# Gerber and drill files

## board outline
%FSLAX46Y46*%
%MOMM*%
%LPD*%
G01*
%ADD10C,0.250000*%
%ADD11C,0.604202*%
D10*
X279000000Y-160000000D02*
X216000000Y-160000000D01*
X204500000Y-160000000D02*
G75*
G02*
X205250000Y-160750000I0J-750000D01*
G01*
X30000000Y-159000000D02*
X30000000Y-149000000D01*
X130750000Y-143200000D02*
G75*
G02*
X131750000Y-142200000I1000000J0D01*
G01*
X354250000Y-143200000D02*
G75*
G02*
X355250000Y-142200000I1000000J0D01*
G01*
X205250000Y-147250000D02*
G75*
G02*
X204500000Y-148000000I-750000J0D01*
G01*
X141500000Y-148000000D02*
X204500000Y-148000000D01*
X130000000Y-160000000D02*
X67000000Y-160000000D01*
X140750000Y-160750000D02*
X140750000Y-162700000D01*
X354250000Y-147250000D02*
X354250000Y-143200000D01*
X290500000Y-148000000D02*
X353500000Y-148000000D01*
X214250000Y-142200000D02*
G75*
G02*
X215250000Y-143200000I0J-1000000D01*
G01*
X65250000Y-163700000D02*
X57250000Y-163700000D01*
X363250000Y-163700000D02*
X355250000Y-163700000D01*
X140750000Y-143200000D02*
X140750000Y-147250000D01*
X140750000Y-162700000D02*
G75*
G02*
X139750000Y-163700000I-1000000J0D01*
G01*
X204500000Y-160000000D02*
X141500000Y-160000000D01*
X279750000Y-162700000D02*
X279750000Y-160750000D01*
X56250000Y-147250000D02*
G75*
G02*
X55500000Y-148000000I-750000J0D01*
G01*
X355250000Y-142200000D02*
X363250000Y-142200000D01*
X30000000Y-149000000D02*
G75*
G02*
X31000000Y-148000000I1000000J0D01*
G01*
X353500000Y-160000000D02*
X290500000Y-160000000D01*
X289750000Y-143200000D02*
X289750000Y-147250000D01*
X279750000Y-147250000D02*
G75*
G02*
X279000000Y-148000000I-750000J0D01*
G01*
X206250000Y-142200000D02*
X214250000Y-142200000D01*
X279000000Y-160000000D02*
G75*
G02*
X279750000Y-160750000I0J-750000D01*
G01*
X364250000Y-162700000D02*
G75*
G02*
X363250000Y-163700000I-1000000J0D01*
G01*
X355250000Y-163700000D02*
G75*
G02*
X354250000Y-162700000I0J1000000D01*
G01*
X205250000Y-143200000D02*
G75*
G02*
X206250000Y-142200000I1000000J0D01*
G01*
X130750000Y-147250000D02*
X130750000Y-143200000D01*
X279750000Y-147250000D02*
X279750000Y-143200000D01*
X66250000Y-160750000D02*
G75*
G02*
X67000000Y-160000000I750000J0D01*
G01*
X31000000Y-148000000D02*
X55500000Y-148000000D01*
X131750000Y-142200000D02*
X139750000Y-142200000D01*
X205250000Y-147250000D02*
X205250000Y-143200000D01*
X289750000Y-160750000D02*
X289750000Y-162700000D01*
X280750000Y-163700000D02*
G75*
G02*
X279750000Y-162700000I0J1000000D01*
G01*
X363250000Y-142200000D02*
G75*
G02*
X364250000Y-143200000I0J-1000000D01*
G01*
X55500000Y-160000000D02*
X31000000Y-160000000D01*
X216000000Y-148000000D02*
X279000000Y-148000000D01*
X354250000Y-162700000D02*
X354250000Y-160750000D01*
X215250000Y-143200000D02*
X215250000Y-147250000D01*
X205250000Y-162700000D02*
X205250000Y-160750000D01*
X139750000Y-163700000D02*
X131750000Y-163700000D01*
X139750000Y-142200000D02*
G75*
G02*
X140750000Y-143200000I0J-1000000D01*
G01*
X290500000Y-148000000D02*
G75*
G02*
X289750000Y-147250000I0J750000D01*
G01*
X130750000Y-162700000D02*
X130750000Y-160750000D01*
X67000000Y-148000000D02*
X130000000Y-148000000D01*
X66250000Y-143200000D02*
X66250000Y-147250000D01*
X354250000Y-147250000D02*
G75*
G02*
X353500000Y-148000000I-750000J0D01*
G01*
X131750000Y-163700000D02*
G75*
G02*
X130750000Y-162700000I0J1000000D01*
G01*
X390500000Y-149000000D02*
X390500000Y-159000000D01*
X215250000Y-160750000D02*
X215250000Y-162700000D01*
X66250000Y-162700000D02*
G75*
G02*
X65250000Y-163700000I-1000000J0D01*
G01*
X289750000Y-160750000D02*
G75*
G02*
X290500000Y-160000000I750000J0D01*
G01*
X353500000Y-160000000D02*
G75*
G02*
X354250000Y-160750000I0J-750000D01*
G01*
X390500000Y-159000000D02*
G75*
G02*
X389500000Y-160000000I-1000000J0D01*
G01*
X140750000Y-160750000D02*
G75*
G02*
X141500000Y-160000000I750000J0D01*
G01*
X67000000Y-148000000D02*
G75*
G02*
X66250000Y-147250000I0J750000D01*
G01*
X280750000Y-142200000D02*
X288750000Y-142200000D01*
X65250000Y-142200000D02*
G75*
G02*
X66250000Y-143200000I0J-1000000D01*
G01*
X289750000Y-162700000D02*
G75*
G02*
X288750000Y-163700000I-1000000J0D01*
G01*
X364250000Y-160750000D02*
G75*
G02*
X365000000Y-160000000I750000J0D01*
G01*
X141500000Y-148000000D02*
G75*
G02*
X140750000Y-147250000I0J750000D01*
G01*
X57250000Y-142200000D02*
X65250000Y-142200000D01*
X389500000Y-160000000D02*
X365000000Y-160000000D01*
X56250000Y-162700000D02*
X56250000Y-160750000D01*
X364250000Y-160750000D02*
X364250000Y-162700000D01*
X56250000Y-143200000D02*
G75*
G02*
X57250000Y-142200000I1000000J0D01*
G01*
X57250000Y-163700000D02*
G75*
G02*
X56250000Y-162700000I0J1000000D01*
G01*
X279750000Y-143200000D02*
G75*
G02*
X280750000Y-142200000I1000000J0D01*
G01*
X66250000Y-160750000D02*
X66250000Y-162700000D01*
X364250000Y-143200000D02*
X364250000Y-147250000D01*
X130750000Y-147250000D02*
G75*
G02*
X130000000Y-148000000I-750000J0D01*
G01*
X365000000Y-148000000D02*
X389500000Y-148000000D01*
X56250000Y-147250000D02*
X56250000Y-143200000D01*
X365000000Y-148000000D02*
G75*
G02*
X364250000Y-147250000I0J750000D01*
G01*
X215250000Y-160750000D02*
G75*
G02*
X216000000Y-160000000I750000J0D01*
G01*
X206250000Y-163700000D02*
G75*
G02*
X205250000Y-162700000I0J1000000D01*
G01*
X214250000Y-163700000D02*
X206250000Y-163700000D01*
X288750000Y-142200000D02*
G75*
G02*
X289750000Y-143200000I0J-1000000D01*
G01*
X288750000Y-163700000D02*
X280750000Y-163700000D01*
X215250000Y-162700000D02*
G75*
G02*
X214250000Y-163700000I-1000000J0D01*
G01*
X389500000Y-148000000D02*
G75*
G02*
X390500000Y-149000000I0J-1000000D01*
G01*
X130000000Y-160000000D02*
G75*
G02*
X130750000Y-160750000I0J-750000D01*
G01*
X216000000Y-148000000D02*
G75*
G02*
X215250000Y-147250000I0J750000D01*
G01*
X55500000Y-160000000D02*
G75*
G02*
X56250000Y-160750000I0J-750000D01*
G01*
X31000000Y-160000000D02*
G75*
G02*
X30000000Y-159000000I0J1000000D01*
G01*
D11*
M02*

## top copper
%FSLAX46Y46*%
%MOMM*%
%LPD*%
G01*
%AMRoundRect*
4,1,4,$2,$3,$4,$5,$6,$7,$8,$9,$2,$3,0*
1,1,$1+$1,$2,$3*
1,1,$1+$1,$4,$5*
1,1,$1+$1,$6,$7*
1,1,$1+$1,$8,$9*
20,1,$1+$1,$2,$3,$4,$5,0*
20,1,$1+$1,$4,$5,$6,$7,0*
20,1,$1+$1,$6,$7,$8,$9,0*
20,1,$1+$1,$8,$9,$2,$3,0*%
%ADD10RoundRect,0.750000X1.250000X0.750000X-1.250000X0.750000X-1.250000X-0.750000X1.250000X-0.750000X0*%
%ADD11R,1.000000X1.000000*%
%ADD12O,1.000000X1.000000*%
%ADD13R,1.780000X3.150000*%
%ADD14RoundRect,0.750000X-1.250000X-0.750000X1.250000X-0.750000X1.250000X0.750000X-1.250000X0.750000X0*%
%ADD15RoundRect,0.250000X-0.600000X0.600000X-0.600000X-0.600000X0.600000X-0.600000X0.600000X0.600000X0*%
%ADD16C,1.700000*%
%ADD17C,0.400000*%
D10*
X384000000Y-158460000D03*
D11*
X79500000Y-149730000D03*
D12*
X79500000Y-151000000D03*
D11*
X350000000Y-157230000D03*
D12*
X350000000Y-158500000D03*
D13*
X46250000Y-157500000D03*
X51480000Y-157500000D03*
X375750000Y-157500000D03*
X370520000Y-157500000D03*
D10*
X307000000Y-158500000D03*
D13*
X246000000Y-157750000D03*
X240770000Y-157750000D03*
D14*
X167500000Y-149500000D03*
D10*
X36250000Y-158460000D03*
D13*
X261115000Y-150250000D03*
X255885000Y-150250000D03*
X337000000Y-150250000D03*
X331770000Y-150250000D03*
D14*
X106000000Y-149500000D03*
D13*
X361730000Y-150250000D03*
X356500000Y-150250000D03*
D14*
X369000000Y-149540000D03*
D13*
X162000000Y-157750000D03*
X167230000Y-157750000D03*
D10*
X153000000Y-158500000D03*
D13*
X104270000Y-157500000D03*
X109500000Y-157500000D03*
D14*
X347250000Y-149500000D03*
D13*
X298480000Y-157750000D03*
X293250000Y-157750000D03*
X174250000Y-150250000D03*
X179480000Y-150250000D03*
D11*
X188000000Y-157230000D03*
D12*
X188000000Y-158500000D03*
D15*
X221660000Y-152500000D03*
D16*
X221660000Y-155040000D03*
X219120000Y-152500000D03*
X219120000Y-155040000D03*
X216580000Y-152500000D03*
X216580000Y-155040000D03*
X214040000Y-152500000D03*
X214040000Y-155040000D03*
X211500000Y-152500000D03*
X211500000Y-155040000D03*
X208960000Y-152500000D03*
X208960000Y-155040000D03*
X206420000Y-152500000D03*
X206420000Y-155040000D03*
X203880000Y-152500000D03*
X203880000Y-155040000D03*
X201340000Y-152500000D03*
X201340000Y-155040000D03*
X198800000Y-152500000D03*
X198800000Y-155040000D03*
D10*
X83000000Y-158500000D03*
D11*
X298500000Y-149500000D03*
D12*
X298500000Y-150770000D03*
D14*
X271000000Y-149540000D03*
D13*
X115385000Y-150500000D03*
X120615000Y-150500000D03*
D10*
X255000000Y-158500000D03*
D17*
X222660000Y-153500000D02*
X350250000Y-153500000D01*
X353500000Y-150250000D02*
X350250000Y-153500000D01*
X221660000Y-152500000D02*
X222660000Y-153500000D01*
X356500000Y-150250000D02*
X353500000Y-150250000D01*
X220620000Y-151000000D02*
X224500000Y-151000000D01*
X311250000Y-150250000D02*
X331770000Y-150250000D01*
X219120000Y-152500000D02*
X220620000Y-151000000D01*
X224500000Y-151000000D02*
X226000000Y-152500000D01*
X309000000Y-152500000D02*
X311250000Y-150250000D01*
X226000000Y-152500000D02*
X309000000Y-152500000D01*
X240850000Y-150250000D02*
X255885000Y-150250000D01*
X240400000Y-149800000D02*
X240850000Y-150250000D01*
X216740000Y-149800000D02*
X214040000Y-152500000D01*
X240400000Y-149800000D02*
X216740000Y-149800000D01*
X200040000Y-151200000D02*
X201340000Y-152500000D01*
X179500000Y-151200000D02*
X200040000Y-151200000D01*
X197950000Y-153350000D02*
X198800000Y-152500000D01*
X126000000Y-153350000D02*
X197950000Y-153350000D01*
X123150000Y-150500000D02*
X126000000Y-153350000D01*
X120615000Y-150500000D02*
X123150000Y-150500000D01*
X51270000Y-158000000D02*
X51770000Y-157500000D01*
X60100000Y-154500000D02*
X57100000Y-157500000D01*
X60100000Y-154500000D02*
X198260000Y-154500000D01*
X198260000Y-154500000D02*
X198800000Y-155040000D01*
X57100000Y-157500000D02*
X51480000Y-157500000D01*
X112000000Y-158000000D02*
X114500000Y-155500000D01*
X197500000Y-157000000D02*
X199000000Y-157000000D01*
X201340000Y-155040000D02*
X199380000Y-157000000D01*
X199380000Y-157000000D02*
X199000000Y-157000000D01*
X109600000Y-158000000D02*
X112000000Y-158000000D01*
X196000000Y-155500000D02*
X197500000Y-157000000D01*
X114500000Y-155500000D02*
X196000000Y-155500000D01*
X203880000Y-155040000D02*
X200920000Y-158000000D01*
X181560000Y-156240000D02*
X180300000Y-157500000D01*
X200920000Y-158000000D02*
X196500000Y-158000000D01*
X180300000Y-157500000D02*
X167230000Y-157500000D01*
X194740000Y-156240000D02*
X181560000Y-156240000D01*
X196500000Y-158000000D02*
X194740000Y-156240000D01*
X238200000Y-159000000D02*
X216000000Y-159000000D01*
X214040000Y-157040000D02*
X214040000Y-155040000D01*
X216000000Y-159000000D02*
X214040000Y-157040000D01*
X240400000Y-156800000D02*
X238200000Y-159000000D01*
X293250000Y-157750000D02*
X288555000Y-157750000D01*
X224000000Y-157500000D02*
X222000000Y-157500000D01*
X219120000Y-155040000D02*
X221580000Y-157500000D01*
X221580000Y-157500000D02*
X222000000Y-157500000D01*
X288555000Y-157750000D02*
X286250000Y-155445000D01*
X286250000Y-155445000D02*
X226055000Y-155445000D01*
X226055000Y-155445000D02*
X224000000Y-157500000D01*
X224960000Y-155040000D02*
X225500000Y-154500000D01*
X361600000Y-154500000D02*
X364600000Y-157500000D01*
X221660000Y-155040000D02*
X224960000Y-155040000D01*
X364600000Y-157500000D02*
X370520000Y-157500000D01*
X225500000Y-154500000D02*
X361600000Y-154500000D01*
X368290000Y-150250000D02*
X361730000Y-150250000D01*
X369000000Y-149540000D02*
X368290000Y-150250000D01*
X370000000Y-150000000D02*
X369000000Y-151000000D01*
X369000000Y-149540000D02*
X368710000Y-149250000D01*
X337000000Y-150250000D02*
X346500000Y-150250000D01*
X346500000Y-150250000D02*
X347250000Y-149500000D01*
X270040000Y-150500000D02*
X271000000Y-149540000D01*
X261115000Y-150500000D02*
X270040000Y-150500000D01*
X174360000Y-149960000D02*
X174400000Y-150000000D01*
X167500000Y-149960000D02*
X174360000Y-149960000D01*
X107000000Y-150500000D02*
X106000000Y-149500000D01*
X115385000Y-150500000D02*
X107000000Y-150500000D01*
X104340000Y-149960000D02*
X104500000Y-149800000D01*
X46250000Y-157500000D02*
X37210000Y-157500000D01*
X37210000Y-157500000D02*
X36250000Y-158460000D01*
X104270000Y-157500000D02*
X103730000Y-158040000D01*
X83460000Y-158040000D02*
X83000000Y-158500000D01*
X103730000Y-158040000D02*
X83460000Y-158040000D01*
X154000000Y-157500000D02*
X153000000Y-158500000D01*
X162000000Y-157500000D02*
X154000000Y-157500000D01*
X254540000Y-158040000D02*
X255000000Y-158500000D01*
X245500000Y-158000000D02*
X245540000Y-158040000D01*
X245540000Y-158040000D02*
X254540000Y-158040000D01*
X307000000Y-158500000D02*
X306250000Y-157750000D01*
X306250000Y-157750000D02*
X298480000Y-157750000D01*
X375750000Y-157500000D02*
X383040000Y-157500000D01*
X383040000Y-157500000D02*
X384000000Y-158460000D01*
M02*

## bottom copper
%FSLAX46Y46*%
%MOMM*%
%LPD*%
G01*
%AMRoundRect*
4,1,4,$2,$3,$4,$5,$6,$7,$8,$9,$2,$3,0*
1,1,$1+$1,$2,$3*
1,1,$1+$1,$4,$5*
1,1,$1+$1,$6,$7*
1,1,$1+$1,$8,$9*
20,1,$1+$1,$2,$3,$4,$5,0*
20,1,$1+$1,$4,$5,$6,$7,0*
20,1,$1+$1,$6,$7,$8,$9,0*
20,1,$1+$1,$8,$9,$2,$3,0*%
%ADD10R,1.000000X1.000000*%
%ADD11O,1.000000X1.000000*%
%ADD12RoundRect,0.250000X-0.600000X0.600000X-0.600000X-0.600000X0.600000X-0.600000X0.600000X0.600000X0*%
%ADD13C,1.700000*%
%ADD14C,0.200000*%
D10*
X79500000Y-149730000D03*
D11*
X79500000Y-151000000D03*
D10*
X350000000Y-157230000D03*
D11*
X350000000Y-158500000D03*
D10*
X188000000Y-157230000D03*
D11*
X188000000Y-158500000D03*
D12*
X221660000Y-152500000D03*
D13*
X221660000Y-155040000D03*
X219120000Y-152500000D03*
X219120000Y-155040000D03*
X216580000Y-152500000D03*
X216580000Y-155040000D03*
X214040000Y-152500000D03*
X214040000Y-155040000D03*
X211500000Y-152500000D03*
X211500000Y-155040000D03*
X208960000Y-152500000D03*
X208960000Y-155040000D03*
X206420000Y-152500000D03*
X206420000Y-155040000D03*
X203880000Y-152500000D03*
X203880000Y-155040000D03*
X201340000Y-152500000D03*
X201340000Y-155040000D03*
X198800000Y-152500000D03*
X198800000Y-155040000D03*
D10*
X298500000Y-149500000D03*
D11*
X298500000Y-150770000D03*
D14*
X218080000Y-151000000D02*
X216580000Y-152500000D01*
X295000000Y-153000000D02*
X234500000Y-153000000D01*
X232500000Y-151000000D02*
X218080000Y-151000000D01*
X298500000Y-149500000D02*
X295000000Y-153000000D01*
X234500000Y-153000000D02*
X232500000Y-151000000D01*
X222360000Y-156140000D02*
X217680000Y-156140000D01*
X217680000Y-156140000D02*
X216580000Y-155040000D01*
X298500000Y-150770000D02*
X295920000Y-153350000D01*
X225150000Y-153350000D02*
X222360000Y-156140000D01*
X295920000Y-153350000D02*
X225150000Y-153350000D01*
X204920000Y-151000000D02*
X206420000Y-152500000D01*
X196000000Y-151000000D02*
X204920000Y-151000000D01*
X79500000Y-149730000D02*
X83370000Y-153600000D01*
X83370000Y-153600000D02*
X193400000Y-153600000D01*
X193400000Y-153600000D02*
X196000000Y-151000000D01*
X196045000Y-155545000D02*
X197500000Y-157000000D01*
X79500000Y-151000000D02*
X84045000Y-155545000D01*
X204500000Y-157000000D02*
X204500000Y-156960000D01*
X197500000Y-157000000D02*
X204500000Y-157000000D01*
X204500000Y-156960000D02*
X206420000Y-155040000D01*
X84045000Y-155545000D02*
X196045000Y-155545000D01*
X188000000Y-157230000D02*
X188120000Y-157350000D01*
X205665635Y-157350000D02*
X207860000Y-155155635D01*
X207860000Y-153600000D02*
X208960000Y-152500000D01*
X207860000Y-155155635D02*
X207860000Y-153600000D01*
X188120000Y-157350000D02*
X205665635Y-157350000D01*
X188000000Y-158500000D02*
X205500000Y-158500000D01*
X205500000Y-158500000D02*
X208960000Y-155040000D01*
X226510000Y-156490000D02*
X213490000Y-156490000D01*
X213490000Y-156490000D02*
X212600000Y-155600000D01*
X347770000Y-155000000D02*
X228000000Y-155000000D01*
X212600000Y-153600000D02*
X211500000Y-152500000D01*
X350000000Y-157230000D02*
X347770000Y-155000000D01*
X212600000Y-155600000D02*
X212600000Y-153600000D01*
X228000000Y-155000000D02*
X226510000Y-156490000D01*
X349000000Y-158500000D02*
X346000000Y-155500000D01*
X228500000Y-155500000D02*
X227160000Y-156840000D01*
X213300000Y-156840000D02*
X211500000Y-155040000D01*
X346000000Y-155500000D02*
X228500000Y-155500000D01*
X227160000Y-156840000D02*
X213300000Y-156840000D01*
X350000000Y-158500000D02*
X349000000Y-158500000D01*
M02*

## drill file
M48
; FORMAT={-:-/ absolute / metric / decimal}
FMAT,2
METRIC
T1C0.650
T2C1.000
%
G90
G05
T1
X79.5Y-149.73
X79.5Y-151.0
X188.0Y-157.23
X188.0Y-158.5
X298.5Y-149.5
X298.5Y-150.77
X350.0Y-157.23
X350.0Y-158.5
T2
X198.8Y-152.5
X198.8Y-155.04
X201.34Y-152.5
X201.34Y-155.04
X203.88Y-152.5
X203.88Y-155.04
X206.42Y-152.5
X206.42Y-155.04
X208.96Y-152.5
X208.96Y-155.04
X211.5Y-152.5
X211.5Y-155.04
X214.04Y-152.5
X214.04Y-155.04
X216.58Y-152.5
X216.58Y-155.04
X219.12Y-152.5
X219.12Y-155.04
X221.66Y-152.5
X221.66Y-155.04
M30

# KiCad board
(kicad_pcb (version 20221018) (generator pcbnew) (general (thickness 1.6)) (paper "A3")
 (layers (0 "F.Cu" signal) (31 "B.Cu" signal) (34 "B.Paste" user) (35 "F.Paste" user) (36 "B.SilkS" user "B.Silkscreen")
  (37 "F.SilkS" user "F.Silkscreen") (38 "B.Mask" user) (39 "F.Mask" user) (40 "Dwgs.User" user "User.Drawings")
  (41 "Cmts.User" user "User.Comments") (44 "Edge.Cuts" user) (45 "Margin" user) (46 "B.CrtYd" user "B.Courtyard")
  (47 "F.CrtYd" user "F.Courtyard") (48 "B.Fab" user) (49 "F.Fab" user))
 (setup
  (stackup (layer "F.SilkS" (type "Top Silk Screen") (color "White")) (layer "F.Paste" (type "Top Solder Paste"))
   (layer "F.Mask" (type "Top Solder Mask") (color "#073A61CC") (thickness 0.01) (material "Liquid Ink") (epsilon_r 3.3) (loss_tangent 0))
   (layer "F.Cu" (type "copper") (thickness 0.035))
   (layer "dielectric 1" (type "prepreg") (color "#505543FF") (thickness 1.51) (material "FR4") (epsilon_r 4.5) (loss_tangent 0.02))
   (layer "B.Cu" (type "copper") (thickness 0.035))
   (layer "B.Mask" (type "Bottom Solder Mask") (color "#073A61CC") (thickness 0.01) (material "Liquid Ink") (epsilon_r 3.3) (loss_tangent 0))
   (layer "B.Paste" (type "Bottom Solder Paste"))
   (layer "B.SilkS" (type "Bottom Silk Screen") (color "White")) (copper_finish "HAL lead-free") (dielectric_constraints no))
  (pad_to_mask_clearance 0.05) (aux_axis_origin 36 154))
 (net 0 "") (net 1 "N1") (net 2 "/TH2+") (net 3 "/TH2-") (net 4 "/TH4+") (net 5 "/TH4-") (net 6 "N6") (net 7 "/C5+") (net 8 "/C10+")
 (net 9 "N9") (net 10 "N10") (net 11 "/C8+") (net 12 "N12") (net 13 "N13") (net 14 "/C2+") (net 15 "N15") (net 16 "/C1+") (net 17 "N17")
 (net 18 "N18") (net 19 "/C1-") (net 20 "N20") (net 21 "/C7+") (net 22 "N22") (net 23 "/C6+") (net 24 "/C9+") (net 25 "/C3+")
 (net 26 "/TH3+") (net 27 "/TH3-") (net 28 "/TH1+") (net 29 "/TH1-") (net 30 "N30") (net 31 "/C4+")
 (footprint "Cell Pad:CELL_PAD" (layer "F.Cu") (at 384 158.46 180)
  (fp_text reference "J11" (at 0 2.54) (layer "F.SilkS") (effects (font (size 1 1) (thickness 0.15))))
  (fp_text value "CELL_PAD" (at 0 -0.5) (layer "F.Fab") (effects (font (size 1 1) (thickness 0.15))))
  (pad "1" smd roundrect (at 0 0 180) (size 4 3) (layers "F.Cu" "F.Paste" "F.Mask") (roundrect_rratio 0.25) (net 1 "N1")))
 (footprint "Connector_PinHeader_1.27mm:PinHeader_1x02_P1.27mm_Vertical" (layer "F.Cu") (at 79.5 149.73)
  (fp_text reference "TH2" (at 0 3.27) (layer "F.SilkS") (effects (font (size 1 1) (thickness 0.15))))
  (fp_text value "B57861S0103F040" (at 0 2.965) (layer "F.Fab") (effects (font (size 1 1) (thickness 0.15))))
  (pad "1" thru_hole rect (at 0 0) (size 1 1) (drill 0.65) (layers "*.Cu" "*.Mask") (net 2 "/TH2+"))
  (pad "2" thru_hole oval (at 0 1.27) (size 1 1) (drill 0.65) (layers "*.Cu" "*.Mask") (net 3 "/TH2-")))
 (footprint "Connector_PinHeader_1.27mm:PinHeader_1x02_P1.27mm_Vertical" (layer "F.Cu") (at 350 157.23)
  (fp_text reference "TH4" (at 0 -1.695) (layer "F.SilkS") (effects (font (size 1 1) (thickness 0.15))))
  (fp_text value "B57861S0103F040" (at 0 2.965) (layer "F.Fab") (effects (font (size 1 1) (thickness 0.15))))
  (pad "1" thru_hole rect (at 0 0) (size 1 1) (drill 0.65) (layers "*.Cu" "*.Mask") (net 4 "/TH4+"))
  (pad "2" thru_hole oval (at 0 1.27) (size 1 1) (drill 0.65) (layers "*.Cu" "*.Mask") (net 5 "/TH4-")))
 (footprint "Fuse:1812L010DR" (layer "F.Cu") (at 48.865 157.5)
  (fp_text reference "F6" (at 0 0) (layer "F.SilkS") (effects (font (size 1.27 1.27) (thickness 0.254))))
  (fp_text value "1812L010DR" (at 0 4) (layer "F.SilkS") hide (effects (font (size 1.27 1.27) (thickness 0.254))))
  (pad "1" smd rect (at -2.615 0) (size 1.78 3.15) (layers "F.Cu" "F.Paste" "F.Mask") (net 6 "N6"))
  (pad "2" smd rect (at 2.615 0) (size 1.78 3.15) (layers "F.Cu" "F.Paste" "F.Mask") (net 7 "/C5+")))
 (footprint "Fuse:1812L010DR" (layer "F.Cu") (at 373.135 157.5 180)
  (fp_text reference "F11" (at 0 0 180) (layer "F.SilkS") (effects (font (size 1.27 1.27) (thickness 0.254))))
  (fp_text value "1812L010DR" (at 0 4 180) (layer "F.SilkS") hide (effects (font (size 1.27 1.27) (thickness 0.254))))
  (pad "1" smd rect (at -2.615 0 180) (size 1.78 3.15) (layers "F.Cu" "F.Paste" "F.Mask") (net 1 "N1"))
  (pad "2" smd rect (at 2.615 0 180) (size 1.78 3.15) (layers "F.Cu" "F.Paste" "F.Mask") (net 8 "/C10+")))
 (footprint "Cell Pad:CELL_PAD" (layer "F.Cu") (at 307 158.5 180)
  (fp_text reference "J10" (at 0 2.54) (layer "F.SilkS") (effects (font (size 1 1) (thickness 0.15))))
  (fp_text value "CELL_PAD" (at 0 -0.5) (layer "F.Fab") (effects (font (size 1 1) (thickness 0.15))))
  (pad "1" smd roundrect (at 0 0 180) (size 4 3) (layers "F.Cu" "F.Paste" "F.Mask") (roundrect_rratio 0.25) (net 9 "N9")))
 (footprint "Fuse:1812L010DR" (layer "F.Cu") (at 243.385 157.75 180)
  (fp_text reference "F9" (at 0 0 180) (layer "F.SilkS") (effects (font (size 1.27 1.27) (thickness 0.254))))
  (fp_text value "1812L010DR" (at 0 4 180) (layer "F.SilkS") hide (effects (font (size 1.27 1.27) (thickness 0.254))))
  (pad "1" smd rect (at -2.615 0 180) (size 1.78 3.15) (layers "F.Cu" "F.Paste" "F.Mask") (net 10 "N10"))
  (pad "2" smd rect (at 2.615 0 180) (size 1.78 3.15) (layers "F.Cu" "F.Paste" "F.Mask") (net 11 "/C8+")))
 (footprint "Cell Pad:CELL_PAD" (layer "F.Cu") (at 167.5 149.5)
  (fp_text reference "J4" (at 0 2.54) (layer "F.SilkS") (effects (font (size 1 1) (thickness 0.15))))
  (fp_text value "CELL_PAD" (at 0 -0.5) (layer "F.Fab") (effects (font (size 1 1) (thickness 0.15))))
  (pad "1" smd roundrect (at 0 0) (size 4 3) (layers "F.Cu" "F.Paste" "F.Mask") (roundrect_rratio 0.25) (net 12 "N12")))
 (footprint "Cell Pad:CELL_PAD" (layer "F.Cu") (at 36.25 158.46 180)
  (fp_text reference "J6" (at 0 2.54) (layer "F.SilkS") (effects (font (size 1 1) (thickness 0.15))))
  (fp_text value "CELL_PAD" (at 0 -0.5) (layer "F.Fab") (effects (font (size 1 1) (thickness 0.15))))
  (pad "1" smd roundrect (at 0 0 180) (size 4 3) (layers "F.Cu" "F.Paste" "F.Mask") (roundrect_rratio 0.25) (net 6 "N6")))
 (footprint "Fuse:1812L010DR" (layer "F.Cu") (at 258.5 150.25 180)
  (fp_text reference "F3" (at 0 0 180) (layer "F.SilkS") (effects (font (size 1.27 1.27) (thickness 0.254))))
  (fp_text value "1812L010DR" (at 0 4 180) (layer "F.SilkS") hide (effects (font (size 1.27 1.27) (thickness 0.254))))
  (pad "1" smd rect (at -2.615 0 180) (size 1.78 3.15) (layers "F.Cu" "F.Paste" "F.Mask") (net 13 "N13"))
  (pad "2" smd rect (at 2.615 0 180) (size 1.78 3.15) (layers "F.Cu" "F.Paste" "F.Mask") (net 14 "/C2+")))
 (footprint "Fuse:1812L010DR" (layer "F.Cu") (at 334.385 150.25 180)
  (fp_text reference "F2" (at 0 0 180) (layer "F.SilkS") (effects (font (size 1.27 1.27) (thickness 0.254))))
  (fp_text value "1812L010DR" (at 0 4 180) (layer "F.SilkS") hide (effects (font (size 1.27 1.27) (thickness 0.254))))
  (pad "1" smd rect (at -2.615 0 180) (size 1.78 3.15) (layers "F.Cu" "F.Paste" "F.Mask") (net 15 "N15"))
  (pad "2" smd rect (at 2.615 0 180) (size 1.78 3.15) (layers "F.Cu" "F.Paste" "F.Mask") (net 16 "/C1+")))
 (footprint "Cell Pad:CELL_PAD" (layer "F.Cu") (at 106 149.5)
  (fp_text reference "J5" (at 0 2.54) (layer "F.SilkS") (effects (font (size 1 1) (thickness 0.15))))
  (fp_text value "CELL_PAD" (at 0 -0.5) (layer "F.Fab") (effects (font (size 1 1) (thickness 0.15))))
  (pad "1" smd roundrect (at 0 0) (size 4 3) (layers "F.Cu" "F.Paste" "F.Mask") (roundrect_rratio 0.25) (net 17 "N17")))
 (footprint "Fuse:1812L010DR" (layer "F.Cu") (at 359.115 150.25 180)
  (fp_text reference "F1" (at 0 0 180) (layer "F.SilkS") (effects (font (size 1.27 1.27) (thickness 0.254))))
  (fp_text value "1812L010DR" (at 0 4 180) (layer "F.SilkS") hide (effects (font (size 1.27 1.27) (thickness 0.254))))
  (pad "1" smd rect (at -2.615 0 180) (size 1.78 3.15) (layers "F.Cu" "F.Paste" "F.Mask") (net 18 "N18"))
  (pad "2" smd rect (at 2.615 0 180) (size 1.78 3.15) (layers "F.Cu" "F.Paste" "F.Mask") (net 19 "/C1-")))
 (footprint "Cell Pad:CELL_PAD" (layer "F.Cu") (at 369 149.54)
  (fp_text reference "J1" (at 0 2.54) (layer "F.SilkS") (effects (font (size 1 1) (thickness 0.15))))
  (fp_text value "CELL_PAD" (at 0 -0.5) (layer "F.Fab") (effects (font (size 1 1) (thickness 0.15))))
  (pad "1" smd roundrect (at 0 0) (size 4 3) (layers "F.Cu" "F.Paste" "F.Mask") (roundrect_rratio 0.25) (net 18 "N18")))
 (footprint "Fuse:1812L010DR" (layer "F.Cu") (at 164.615 157.75)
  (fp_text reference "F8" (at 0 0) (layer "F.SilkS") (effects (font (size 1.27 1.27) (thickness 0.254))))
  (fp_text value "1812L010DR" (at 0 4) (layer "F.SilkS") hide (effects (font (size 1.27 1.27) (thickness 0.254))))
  (pad "1" smd rect (at -2.615 0) (size 1.78 3.15) (layers "F.Cu" "F.Paste" "F.Mask") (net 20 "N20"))
  (pad "2" smd rect (at 2.615 0) (size 1.78 3.15) (layers "F.Cu" "F.Paste" "F.Mask") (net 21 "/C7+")))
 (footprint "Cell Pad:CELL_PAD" (layer "F.Cu") (at 153 158.5 180)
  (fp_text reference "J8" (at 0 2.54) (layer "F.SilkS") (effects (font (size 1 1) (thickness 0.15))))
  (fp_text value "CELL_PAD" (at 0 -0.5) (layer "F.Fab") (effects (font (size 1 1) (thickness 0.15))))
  (pad "1" smd roundrect (at 0 0 180) (size 4 3) (layers "F.Cu" "F.Paste" "F.Mask") (roundrect_rratio 0.25) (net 20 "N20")))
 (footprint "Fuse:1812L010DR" (layer "F.Cu") (at 106.885 157.5)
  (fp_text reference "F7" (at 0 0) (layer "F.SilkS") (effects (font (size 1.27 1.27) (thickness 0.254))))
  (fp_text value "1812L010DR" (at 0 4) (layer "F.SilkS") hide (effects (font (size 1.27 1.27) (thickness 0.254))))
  (pad "1" smd rect (at -2.615 0) (size 1.78 3.15) (layers "F.Cu" "F.Paste" "F.Mask") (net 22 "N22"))
  (pad "2" smd rect (at 2.615 0) (size 1.78 3.15) (layers "F.Cu" "F.Paste" "F.Mask") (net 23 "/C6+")))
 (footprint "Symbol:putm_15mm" (layer "F.Cu") (at 136 154)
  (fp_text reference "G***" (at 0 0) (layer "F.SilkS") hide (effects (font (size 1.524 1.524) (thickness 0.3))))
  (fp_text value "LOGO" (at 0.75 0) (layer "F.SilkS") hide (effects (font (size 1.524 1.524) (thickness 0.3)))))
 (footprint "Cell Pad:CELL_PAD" (layer "F.Cu") (at 347.25 149.5)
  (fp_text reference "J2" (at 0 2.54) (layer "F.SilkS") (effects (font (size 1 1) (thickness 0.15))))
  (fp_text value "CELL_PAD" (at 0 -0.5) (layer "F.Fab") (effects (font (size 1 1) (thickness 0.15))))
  (pad "1" smd roundrect (at 0 0) (size 4 3) (layers "F.Cu" "F.Paste" "F.Mask") (roundrect_rratio 0.25) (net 15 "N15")))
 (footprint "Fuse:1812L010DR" (layer "F.Cu") (at 295.865 157.75 180)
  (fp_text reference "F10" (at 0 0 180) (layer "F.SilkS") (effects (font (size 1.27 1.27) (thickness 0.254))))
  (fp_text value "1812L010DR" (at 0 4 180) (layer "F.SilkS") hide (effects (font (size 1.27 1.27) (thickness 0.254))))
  (pad "1" smd rect (at -2.615 0 180) (size 1.78 3.15) (layers "F.Cu" "F.Paste" "F.Mask") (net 9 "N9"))
  (pad "2" smd rect (at 2.615 0 180) (size 1.78 3.15) (layers "F.Cu" "F.Paste" "F.Mask") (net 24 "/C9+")))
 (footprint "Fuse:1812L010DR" (layer "F.Cu") (at 176.865 150.25)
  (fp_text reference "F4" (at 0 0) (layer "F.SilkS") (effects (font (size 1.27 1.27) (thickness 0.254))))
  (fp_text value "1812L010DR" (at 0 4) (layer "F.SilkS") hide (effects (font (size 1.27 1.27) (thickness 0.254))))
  (pad "1" smd rect (at -2.615 0) (size 1.78 3.15) (layers "F.Cu" "F.Paste" "F.Mask") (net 12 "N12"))
  (pad "2" smd rect (at 2.615 0) (size 1.78 3.15) (layers "F.Cu" "F.Paste" "F.Mask") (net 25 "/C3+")))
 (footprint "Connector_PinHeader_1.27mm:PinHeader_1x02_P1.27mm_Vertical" (layer "F.Cu") (at 188 157.23)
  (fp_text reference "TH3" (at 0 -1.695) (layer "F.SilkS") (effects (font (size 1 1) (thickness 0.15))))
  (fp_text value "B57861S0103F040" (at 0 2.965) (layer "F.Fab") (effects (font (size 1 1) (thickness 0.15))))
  (pad "1" thru_hole rect (at 0 0) (size 1 1) (drill 0.65) (layers "*.Cu" "*.Mask") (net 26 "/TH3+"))
  (pad "2" thru_hole oval (at 0 1.27) (size 1 1) (drill 0.65) (layers "*.Cu" "*.Mask") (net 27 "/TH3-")))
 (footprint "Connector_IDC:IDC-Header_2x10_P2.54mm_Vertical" (layer "F.Cu") (at 221.66 152.5 -90)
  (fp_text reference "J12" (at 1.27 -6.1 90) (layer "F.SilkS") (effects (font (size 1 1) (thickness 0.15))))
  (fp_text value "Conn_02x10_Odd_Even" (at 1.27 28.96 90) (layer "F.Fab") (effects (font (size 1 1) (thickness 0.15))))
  (pad "1" thru_hole roundrect (at 0 0 270) (size 1.7 1.7) (drill 1) (layers "*.Cu" "*.Mask") (roundrect_rratio 0.147059) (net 19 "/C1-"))
  (pad "2" thru_hole circle (at 2.54 0 270) (size 1.7 1.7) (drill 1) (layers "*.Cu" "*.Mask") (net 8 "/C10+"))
  (pad "3" thru_hole circle (at 0 2.54 270) (size 1.7 1.7) (drill 1) (layers "*.Cu" "*.Mask") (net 16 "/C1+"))
  (pad "4" thru_hole circle (at 2.54 2.54 270) (size 1.7 1.7) (drill 1) (layers "*.Cu" "*.Mask") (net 24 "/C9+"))
  (pad "5" thru_hole circle (at 0 5.08 270) (size 1.7 1.7) (drill 1) (layers "*.Cu" "*.Mask") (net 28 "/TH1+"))
  (pad "6" thru_hole circle (at 2.54 5.08 270) (size 1.7 1.7) (drill 1) (layers "*.Cu" "*.Mask") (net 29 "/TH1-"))
  (pad "7" thru_hole circle (at 0 7.62 270) (size 1.7 1.7) (drill 1) (layers "*.Cu" "*.Mask") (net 14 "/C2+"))
  (pad "8" thru_hole circle (at 2.54 7.62 270) (size 1.7 1.7) (drill 1) (layers "*.Cu" "*.Mask") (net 11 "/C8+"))
  (pad "9" thru_hole circle (at 0 10.16 270) (size 1.7 1.7) (drill 1) (layers "*.Cu" "*.Mask") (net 4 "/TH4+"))
  (pad "10" thru_hole circle (at 2.54 10.16 270) (size 1.7 1.7) (drill 1) (layers "*.Cu" "*.Mask") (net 5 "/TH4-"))
  (pad "11" thru_hole circle (at 0 12.7 270) (size 1.7 1.7) (drill 1) (layers "*.Cu" "*.Mask") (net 26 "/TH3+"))
  (pad "12" thru_hole circle (at 2.54 12.7 270) (size 1.7 1.7) (drill 1) (layers "*.Cu" "*.Mask") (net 27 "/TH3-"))
  (pad "13" thru_hole circle (at 0 15.24 270) (size 1.7 1.7) (drill 1) (layers "*.Cu" "*.Mask") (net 2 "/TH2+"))
  (pad "14" thru_hole circle (at 2.54 15.24 270) (size 1.7 1.7) (drill 1) (layers "*.Cu" "*.Mask") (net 3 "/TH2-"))
  (pad "15" thru_hole circle (at 0 17.78 270) (size 1.7 1.7) (drill 1) (layers "*.Cu" "*.Mask") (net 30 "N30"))
  (pad "16" thru_hole circle (at 2.54 17.78 270) (size 1.7 1.7) (drill 1) (layers "*.Cu" "*.Mask") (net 21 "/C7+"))
  (pad "17" thru_hole circle (at 0 20.32 270) (size 1.7 1.7) (drill 1) (layers "*.Cu" "*.Mask") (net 25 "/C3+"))
  (pad "18" thru_hole circle (at 2.54 20.32 270) (size 1.7 1.7) (drill 1) (layers "*.Cu" "*.Mask") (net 23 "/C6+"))
  (pad "19" thru_hole circle (at 0 22.86 270) (size 1.7 1.7) (drill 1) (layers "*.Cu" "*.Mask") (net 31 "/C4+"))
  (pad "20" thru_hole circle (at 2.54 22.86 270) (size 1.7 1.7) (drill 1) (layers "*.Cu" "*.Mask") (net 7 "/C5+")))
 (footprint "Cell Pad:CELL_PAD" (layer "F.Cu") (at 83 158.5 180)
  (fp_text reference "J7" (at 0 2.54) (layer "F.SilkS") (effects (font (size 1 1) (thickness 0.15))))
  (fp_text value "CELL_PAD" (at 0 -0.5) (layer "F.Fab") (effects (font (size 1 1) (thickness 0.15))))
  (pad "1" smd roundrect (at 0 0 180) (size 4 3) (layers "F.Cu" "F.Paste" "F.Mask") (roundrect_rratio 0.25) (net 22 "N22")))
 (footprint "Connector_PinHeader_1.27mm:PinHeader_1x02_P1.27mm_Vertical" (layer "F.Cu") (at 298.5 149.5)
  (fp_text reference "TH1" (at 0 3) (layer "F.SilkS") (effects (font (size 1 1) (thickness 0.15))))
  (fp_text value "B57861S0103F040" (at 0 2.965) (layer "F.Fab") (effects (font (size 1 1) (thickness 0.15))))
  (pad "1" thru_hole rect (at 0 0) (size 1 1) (drill 0.65) (layers "*.Cu" "*.Mask") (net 28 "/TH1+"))
  (pad "2" thru_hole oval (at 0 1.27) (size 1 1) (drill 0.65) (layers "*.Cu" "*.Mask") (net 29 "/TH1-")))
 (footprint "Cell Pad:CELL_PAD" (layer "F.Cu") (at 271 149.54)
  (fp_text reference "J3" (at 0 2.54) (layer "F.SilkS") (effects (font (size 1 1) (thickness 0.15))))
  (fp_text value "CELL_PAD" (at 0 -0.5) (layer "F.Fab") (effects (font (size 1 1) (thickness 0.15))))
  (pad "1" smd roundrect (at 0 0) (size 4 3) (layers "F.Cu" "F.Paste" "F.Mask") (roundrect_rratio 0.25) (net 13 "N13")))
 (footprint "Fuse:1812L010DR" (layer "F.Cu") (at 118 150.5)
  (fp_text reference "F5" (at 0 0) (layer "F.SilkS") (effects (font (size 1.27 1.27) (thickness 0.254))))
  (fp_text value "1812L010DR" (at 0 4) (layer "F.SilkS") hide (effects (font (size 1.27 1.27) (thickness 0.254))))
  (pad "1" smd rect (at -2.615 0) (size 1.78 3.15) (layers "F.Cu" "F.Paste" "F.Mask") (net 17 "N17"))
  (pad "2" smd rect (at 2.615 0) (size 1.78 3.15) (layers "F.Cu" "F.Paste" "F.Mask") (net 31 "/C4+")))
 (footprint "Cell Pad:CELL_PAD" (layer "F.Cu") (at 255 158.5 180)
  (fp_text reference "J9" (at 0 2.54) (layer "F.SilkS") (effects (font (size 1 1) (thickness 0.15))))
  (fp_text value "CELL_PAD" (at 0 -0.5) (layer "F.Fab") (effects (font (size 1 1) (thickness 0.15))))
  (pad "1" smd roundrect (at 0 0 180) (size 4 3) (layers "F.Cu" "F.Paste" "F.Mask") (roundrect_rratio 0.25) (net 10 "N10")))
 (gr_line (start 279 160) (end 216 160) (stroke (width 0.25) (type solid)) (layer "Edge.Cuts"))
 (gr_arc (start 204.5 160) (mid 205.030317 160.219677) (end 205.25 160.75) (stroke (width 0.25) (type solid)) (layer "Edge.Cuts"))
 (gr_line (start 30 159) (end 30 149) (stroke (width 0.25) (type solid)) (layer "Edge.Cuts"))
 (gr_arc (start 130.75 143.2) (mid 131.042894 142.4929) (end 131.75 142.2) (stroke (width 0.25) (type solid)) (layer "Edge.Cuts"))
 (gr_arc (start 354.25 143.2) (mid 354.542894 142.4929) (end 355.25 142.2) (stroke (width 0.25) (type solid)) (layer "Edge.Cuts"))
 (gr_arc (start 205.25 147.25) (mid 205.030331 147.780337) (end 204.5 148) (stroke (width 0.25) (type solid)) (layer "Edge.Cuts"))
 (gr_line (start 141.5 148) (end 204.5 148) (stroke (width 0.25) (type solid)) (layer "Edge.Cuts"))
 (gr_line (start 130 160) (end 67 160) (stroke (width 0.25) (type solid)) (layer "Edge.Cuts"))
 (gr_line (start 140.75 160.75) (end 140.75 162.7) (stroke (width 0.25) (type solid)) (layer "Edge.Cuts"))
 (gr_line (start 354.25 147.25) (end 354.25 143.2) (stroke (width 0.25) (type solid)) (layer "Edge.Cuts"))
 (gr_line (start 290.5 148) (end 353.5 148) (stroke (width 0.25) (type solid)) (layer "Edge.Cuts"))
 (gr_arc (start 214.25 142.2) (mid 214.957094 142.4929) (end 215.25 143.2) (stroke (width 0.25) (type solid)) (layer "Edge.Cuts"))
 (gr_line (start 65.25 163.7) (end 57.25 163.7) (stroke (width 0.25) (type solid)) (layer "Edge.Cuts"))
 (gr_line (start 363.25 163.7) (end 355.25 163.7) (stroke (width 0.25) (type solid)) (layer "Edge.Cuts"))
 (gr_line (start 140.75 143.2) (end 140.75 147.25) (stroke (width 0.25) (type solid)) (layer "Edge.Cuts"))
 (gr_arc (start 140.75 162.7) (mid 140.457108 163.407114) (end 139.75 163.7) (stroke (width 0.25) (type solid)) (layer "Edge.Cuts"))
 (gr_line (start 204.5 160) (end 141.5 160) (stroke (width 0.25) (type solid)) (layer "Edge.Cuts"))
 (gr_line (start 279.75 162.7) (end 279.75 160.75) (stroke (width 0.25) (type solid)) (layer "Edge.Cuts"))
 (gr_arc (start 56.25 147.25) (mid 56.03033 147.78033) (end 55.5 148) (stroke (width 0.25) (type solid)) (layer "Edge.Cuts"))
 (gr_line (start 355.25 142.2) (end 363.25 142.2) (stroke (width 0.25) (type solid)) (layer "Edge.Cuts"))
 (gr_arc (start 30 149) (mid 30.292894 148.292894) (end 31 148) (stroke (width 0.25) (type solid)) (layer "Edge.Cuts"))
 (gr_line (start 353.5 160) (end 290.5 160) (stroke (width 0.25) (type solid)) (layer "Edge.Cuts"))
 (gr_line (start 289.75 143.2) (end 289.75 147.25) (stroke (width 0.25) (type solid)) (layer "Edge.Cuts"))
 (gr_arc (start 279.75 147.25) (mid 279.530331 147.780337) (end 279 148) (stroke (width 0.25) (type solid)) (layer "Edge.Cuts"))
 (gr_line (start 206.25 142.2) (end 214.25 142.2) (stroke (width 0.25) (type solid)) (layer "Edge.Cuts"))
 (gr_arc (start 279 160) (mid 279.530317 160.219677) (end 279.75 160.75) (stroke (width 0.25) (type solid)) (layer "Edge.Cuts"))
 (gr_arc (start 364.25 162.7) (mid 363.957108 163.407114) (end 363.25 163.7) (stroke (width 0.25) (type solid)) (layer "Edge.Cuts"))
 (gr_arc (start 355.25 163.7) (mid 354.54288 163.407114) (end 354.25 162.7) (stroke (width 0.25) (type solid)) (layer "Edge.Cuts"))
 (gr_arc (start 205.25 143.2) (mid 205.542894 142.4929) (end 206.25 142.2) (stroke (width 0.25) (type solid)) (layer "Edge.Cuts"))
 (gr_line (start 130.75 147.25) (end 130.75 143.2) (stroke (width 0.25) (type solid)) (layer "Edge.Cuts"))
 (gr_line (start 279.75 147.25) (end 279.75 143.2) (stroke (width 0.25) (type solid)) (layer "Edge.Cuts"))
 (gr_arc (start 66.25 160.75) (mid 66.469671 160.219677) (end 67 160) (stroke (width 0.25) (type solid)) (layer "Edge.Cuts"))
 (gr_line (start 31 148) (end 55.5 148) (stroke (width 0.25) (type solid)) (layer "Edge.Cuts"))
 (gr_line (start 131.75 142.2) (end 139.75 142.2) (stroke (width 0.25) (type solid)) (layer "Edge.Cuts"))
 (gr_line (start 205.25 147.25) (end 205.25 143.2) (stroke (width 0.25) (type solid)) (layer "Edge.Cuts"))
 (gr_line (start 289.75 160.75) (end 289.75 162.7) (stroke (width 0.25) (type solid)) (layer "Edge.Cuts"))
 (gr_arc (start 280.75 163.7) (mid 280.04288 163.407114) (end 279.75 162.7) (stroke (width 0.25) (type solid)) (layer "Edge.Cuts"))
 (gr_arc (start 363.25 142.2) (mid 363.957094 142.4929) (end 364.25 143.2) (stroke (width 0.25) (type solid)) (layer "Edge.Cuts"))
 (gr_line (start 55.5 160) (end 31 160) (stroke (width 0.25) (type solid)) (layer "Edge.Cuts"))
 (gr_line (start 216 148) (end 279 148) (stroke (width 0.25) (type solid)) (layer "Edge.Cuts"))
 (gr_line (start 354.25 162.7) (end 354.25 160.75) (stroke (width 0.25) (type solid)) (layer "Edge.Cuts"))
 (gr_line (start 215.25 143.2) (end 215.25 147.25) (stroke (width 0.25) (type solid)) (layer "Edge.Cuts"))
 (gr_line (start 205.25 162.7) (end 205.25 160.75) (stroke (width 0.25) (type solid)) (layer "Edge.Cuts"))
 (gr_line (start 139.75 163.7) (end 131.75 163.7) (stroke (width 0.25) (type solid)) (layer "Edge.Cuts"))
 (gr_arc (start 139.75 142.2) (mid 140.457094 142.4929) (end 140.75 143.2) (stroke (width 0.25) (type solid)) (layer "Edge.Cuts"))
 (gr_arc (start 290.5 148) (mid 289.969657 147.780337) (end 289.75 147.25) (stroke (width 0.25) (type solid)) (layer "Edge.Cuts"))
 (gr_line (start 130.75 162.7) (end 130.75 160.75) (stroke (width 0.25) (type solid)) (layer "Edge.Cuts"))
 (gr_line (start 67 148) (end 130 148) (stroke (width 0.25) (type solid)) (layer "Edge.Cuts"))
 (gr_line (start 66.25 143.2) (end 66.25 147.25) (stroke (width 0.25) (type solid)) (layer "Edge.Cuts"))
 (gr_arc (start 354.25 147.25) (mid 354.030331 147.780337) (end 353.5 148) (stroke (width 0.25) (type solid)) (layer "Edge.Cuts"))
 (gr_arc (start 131.75 163.7) (mid 131.04288 163.407114) (end 130.75 162.7) (stroke (width 0.25) (type solid)) (layer "Edge.Cuts"))
 (gr_line (start 390.5 149) (end 390.5 159) (stroke (width 0.25) (type solid)) (layer "Edge.Cuts"))
 (gr_line (start 215.25 160.75) (end 215.25 162.7) (stroke (width 0.25) (type solid)) (layer "Edge.Cuts"))
 (gr_arc (start 66.25 162.7) (mid 65.957107 163.407107) (end 65.25 163.7) (stroke (width 0.25) (type solid)) (layer "Edge.Cuts"))
 (gr_arc (start 289.75 160.75) (mid 289.969671 160.219677) (end 290.5 160) (stroke (width 0.25) (type solid)) (layer "Edge.Cuts"))
 (gr_arc (start 353.5 160) (mid 354.030317 160.219677) (end 354.25 160.75) (stroke (width 0.25) (type solid)) (layer "Edge.Cuts"))
 (gr_arc (start 390.5 159) (mid 390.207108 159.707114) (end 389.5 160) (stroke (width 0.25) (type solid)) (layer "Edge.Cuts"))
 (gr_arc (start 140.75 160.75) (mid 140.969671 160.219677) (end 141.5 160) (stroke (width 0.25) (type solid)) (layer "Edge.Cuts"))
 (gr_arc (start 67 148) (mid 66.469657 147.780337) (end 66.25 147.25) (stroke (width 0.25) (type solid)) (layer "Edge.Cuts"))
 (gr_line (start 280.75 142.2) (end 288.75 142.2) (stroke (width 0.25) (type solid)) (layer "Edge.Cuts"))
 (gr_arc (start 65.25 142.2) (mid 65.957107 142.492893) (end 66.25 143.2) (stroke (width 0.25) (type solid)) (layer "Edge.Cuts"))
 (gr_arc (start 289.75 162.7) (mid 289.457108 163.407114) (end 288.75 163.7) (stroke (width 0.25) (type solid)) (layer "Edge.Cuts"))
 (gr_arc (start 364.25 160.75) (mid 364.469671 160.219677) (end 365 160) (stroke (width 0.25) (type solid)) (layer "Edge.Cuts"))
 (gr_arc (start 141.5 148) (mid 140.969657 147.780337) (end 140.75 147.25) (stroke (width 0.25) (type solid)) (layer "Edge.Cuts"))
 (gr_line (start 57.25 142.2) (end 65.25 142.2) (stroke (width 0.25) (type solid)) (layer "Edge.Cuts"))
 (gr_line (start 389.5 160) (end 365 160) (stroke (width 0.25) (type solid)) (layer "Edge.Cuts"))
 (gr_line (start 56.25 162.7) (end 56.25 160.75) (stroke (width 0.25) (type solid)) (layer "Edge.Cuts"))
 (gr_line (start 364.25 160.75) (end 364.25 162.7) (stroke (width 0.25) (type solid)) (layer "Edge.Cuts"))
 (gr_arc (start 56.25 143.2) (mid 56.542894 142.492894) (end 57.25 142.2) (stroke (width 0.25) (type solid)) (layer "Edge.Cuts"))
 (gr_arc (start 57.25 163.7) (mid 56.542894 163.407106) (end 56.25 162.7) (stroke (width 0.25) (type solid)) (layer "Edge.Cuts"))
 (gr_arc (start 279.75 143.2) (mid 280.042894 142.4929) (end 280.75 142.2) (stroke (width 0.25) (type solid)) (layer "Edge.Cuts"))
 (gr_line (start 66.25 160.75) (end 66.25 162.7) (stroke (width 0.25) (type solid)) (layer "Edge.Cuts"))
 (gr_line (start 364.25 143.2) (end 364.25 147.25) (stroke (width 0.25) (type solid)) (layer "Edge.Cuts"))
 (gr_arc (start 130.75 147.25) (mid 130.530331 147.780337) (end 130 148) (stroke (width 0.25) (type solid)) (layer "Edge.Cuts"))
 (gr_line (start 365 148) (end 389.5 148) (stroke (width 0.25) (type solid)) (layer "Edge.Cuts"))
 (gr_line (start 56.25 147.25) (end 56.25 143.2) (stroke (width 0.25) (type solid)) (layer "Edge.Cuts"))
 (gr_arc (start 365 148) (mid 364.469657 147.780337) (end 364.25 147.25) (stroke (width 0.25) (type solid)) (layer "Edge.Cuts"))
 (gr_arc (start 215.25 160.75) (mid 215.469671 160.219677) (end 216 160) (stroke (width 0.25) (type solid)) (layer "Edge.Cuts"))
 (gr_arc (start 206.25 163.7) (mid 205.54288 163.407114) (end 205.25 162.7) (stroke (width 0.25) (type solid)) (layer "Edge.Cuts"))
 (gr_line (start 214.25 163.7) (end 206.25 163.7) (stroke (width 0.25) (type solid)) (layer "Edge.Cuts"))
 (gr_arc (start 288.75 142.2) (mid 289.457094 142.4929) (end 289.75 143.2) (stroke (width 0.25) (type solid)) (layer "Edge.Cuts"))
 (gr_line (start 288.75 163.7) (end 280.75 163.7) (stroke (width 0.25) (type solid)) (layer "Edge.Cuts"))
 (gr_arc (start 215.25 162.7) (mid 214.957108 163.407114) (end 214.25 163.7) (stroke (width 0.25) (type solid)) (layer "Edge.Cuts"))
 (gr_arc (start 389.5 148) (mid 390.207094 148.2929) (end 390.5 149) (stroke (width 0.25) (type solid)) (layer "Edge.Cuts"))
 (gr_arc (start 130 160) (mid 130.530317 160.219677) (end 130.75 160.75) (stroke (width 0.25) (type solid)) (layer "Edge.Cuts"))
 (gr_arc (start 216 148) (mid 215.469657 147.780337) (end 215.25 147.25) (stroke (width 0.25) (type solid)) (layer "Edge.Cuts"))
 (gr_arc (start 55.5 160) (mid 56.03033 160.21967) (end 56.25 160.75) (stroke (width 0.25) (type solid)) (layer "Edge.Cuts"))
 (gr_arc (start 31 160) (mid 30.292894 159.707106) (end 30 159) (stroke (width 0.25) (type solid)) (layer "Edge.Cuts"))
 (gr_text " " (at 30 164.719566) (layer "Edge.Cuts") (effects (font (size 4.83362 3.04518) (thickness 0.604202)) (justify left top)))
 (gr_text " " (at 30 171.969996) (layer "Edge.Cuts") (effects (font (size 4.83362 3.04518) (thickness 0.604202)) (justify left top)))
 (segment (start 222.66 153.5) (end 350.25 153.5) (width 0.4) (layer "F.Cu") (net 19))
 (segment (start 353.5 150.25) (end 350.25 153.5) (width 0.4) (layer "F.Cu") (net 19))
 (segment (start 221.66 152.5) (end 222.66 153.5) (width 0.4) (layer "F.Cu") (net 19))
 (segment (start 356.5 150.25) (end 353.5 150.25) (width 0.4) (layer "F.Cu") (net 19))
 (segment (start 220.62 151) (end 224.5 151) (width 0.4) (layer "F.Cu") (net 16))
 (segment (start 311.25 150.25) (end 331.77 150.25) (width 0.4) (layer "F.Cu") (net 16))
 (segment (start 219.12 152.5) (end 220.62 151) (width 0.4) (layer "F.Cu") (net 16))
 (segment (start 224.5 151) (end 226 152.5) (width 0.4) (layer "F.Cu") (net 16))
 (segment (start 309 152.5) (end 311.25 150.25) (width 0.4) (layer "F.Cu") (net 16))
 (segment (start 226 152.5) (end 309 152.5) (width 0.4) (layer "F.Cu") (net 16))
 (segment (start 240.85 150.25) (end 255.885 150.25) (width 0.4) (layer "F.Cu") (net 14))
 (segment (start 240.4 149.8) (end 240.85 150.25) (width 0.4) (layer "F.Cu") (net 14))
 (segment (start 216.74 149.8) (end 214.04 152.5) (width 0.4) (layer "F.Cu") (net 14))
 (segment (start 240.4 149.8) (end 216.74 149.8) (width 0.4) (layer "F.Cu") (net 14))
 (segment (start 200.04 151.2) (end 201.34 152.5) (width 0.4) (layer "F.Cu") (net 25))
 (segment (start 179.5 151.2) (end 200.04 151.2) (width 0.4) (layer "F.Cu") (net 25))
 (segment (start 197.95 153.35) (end 198.8 152.5) (width 0.4) (layer "F.Cu") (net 31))
 (segment (start 126 153.35) (end 197.95 153.35) (width 0.4) (layer "F.Cu") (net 31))
 (segment (start 123.15 150.5) (end 126 153.35) (width 0.4) (layer "F.Cu") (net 31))
 (segment (start 120.615 150.5) (end 123.15 150.5) (width 0.4) (layer "F.Cu") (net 31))
 (segment (start 51.27 158) (end 51.77 157.5) (width 0.4) (layer "F.Cu") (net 7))
 (segment (start 60.1 154.5) (end 57.1 157.5) (width 0.4) (layer "F.Cu") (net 7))
 (segment (start 60.1 154.5) (end 198.26 154.5) (width 0.4) (layer "F.Cu") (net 7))
 (segment (start 198.26 154.5) (end 198.8 155.04) (width 0.4) (layer "F.Cu") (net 7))
 (segment (start 57.1 157.5) (end 51.48 157.5) (width 0.4) (layer "F.Cu") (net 7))
 (segment (start 112 158) (end 114.5 155.5) (width 0.4) (layer "F.Cu") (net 23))
 (segment (start 197.5 157) (end 199 157) (width 0.4) (layer "F.Cu") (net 23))
 (segment (start 201.34 155.04) (end 199.38 157) (width 0.4) (layer "F.Cu") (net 23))
 (segment (start 199.38 157) (end 199 157) (width 0.4) (layer "F.Cu") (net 23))
 (segment (start 109.6 158) (end 112 158) (width 0.4) (layer "F.Cu") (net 23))
 (segment (start 196 155.5) (end 197.5 157) (width 0.4) (layer "F.Cu") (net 23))
 (segment (start 114.5 155.5) (end 196 155.5) (width 0.4) (layer "F.Cu") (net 23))
 (segment (start 203.88 155.04) (end 200.92 158) (width 0.4) (layer "F.Cu") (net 21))
 (segment (start 181.56 156.24) (end 180.3 157.5) (width 0.4) (layer "F.Cu") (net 21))
 (segment (start 200.92 158) (end 196.5 158) (width 0.4) (layer "F.Cu") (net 21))
 (segment (start 180.3 157.5) (end 167.23 157.5) (width 0.4) (layer "F.Cu") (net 21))
 (segment (start 194.74 156.24) (end 181.56 156.24) (width 0.4) (layer "F.Cu") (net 21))
 (segment (start 196.5 158) (end 194.74 156.24) (width 0.4) (layer "F.Cu") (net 21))
 (segment (start 238.2 159) (end 216 159) (width 0.4) (layer "F.Cu") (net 11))
 (segment (start 214.04 157.04) (end 214.04 155.04) (width 0.4) (layer "F.Cu") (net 11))
 (segment (start 216 159) (end 214.04 157.04) (width 0.4) (layer "F.Cu") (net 11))
 (segment (start 240.4 156.8) (end 238.2 159) (width 0.4) (layer "F.Cu") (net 11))
 (segment (start 293.25 157.75) (end 288.555 157.75) (width 0.4) (layer "F.Cu") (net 24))
 (segment (start 224 157.5) (end 222 157.5) (width 0.4) (layer "F.Cu") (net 24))
 (segment (start 219.12 155.04) (end 221.58 157.5) (width 0.4) (layer "F.Cu") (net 24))
 (segment (start 221.58 157.5) (end 222 157.5) (width 0.4) (layer "F.Cu") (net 24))
 (segment (start 288.555 157.75) (end 286.25 155.445) (width 0.4) (layer "F.Cu") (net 24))
 (segment (start 286.25 155.445) (end 226.055 155.445) (width 0.4) (layer "F.Cu") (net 24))
 (segment (start 226.055 155.445) (end 224 157.5) (width 0.4) (layer "F.Cu") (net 24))
 (segment (start 224.96 155.04) (end 225.5 154.5) (width 0.4) (layer "F.Cu") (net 8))
 (segment (start 361.6 154.5) (end 364.6 157.5) (width 0.4) (layer "F.Cu") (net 8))
 (segment (start 221.66 155.04) (end 224.96 155.04) (width 0.4) (layer "F.Cu") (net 8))
 (segment (start 364.6 157.5) (end 370.52 157.5) (width 0.4) (layer "F.Cu") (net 8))
 (segment (start 225.5 154.5) (end 361.6 154.5) (width 0.4) (layer "F.Cu") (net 8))
 (segment (start 218.08 151) (end 216.58 152.5) (width 0.2) (layer "B.Cu") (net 28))
 (segment (start 295 153) (end 234.5 153) (width 0.2) (layer "B.Cu") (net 28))
 (segment (start 232.5 151) (end 218.08 151) (width 0.2) (layer "B.Cu") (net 28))
 (segment (start 298.5 149.5) (end 295 153) (width 0.2) (layer "B.Cu") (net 28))
 (segment (start 234.5 153) (end 232.5 151) (width 0.2) (layer "B.Cu") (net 28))
 (segment (start 222.36 156.14) (end 217.68 156.14) (width 0.2) (layer "B.Cu") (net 29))
 (segment (start 217.68 156.14) (end 216.58 155.04) (width 0.2) (layer "B.Cu") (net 29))
 (segment (start 298.5 150.77) (end 295.92 153.35) (width 0.2) (layer "B.Cu") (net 29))
 (segment (start 225.15 153.35) (end 222.36 156.14) (width 0.2) (layer "B.Cu") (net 29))
 (segment (start 295.92 153.35) (end 225.15 153.35) (width 0.2) (layer "B.Cu") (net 29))
 (segment (start 204.92 151) (end 206.42 152.5) (width 0.2) (layer "B.Cu") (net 2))
 (segment (start 196 151) (end 204.92 151) (width 0.2) (layer "B.Cu") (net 2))
 (segment (start 79.5 149.73) (end 83.37 153.6) (width 0.2) (layer "B.Cu") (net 2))
 (segment (start 83.37 153.6) (end 193.4 153.6) (width 0.2) (layer "B.Cu") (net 2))
 (segment (start 193.4 153.6) (end 196 151) (width 0.2) (layer "B.Cu") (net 2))
 (segment (start 196.045 155.545) (end 197.5 157) (width 0.2) (layer "B.Cu") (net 3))
 (segment (start 79.5 151) (end 84.045 155.545) (width 0.2) (layer "B.Cu") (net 3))
 (segment (start 204.5 157) (end 204.5 156.96) (width 0.2) (layer "B.Cu") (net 3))
 (segment (start 197.5 157) (end 204.5 157) (width 0.2) (layer "B.Cu") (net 3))
 (segment (start 204.5 156.96) (end 206.42 155.04) (width 0.2) (layer "B.Cu") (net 3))
 (segment (start 84.045 155.545) (end 196.045 155.545) (width 0.2) (layer "B.Cu") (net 3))
 (segment (start 188 157.23) (end 188.12 157.35) (width 0.2) (layer "B.Cu") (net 26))
 (segment (start 205.665635 157.35) (end 207.86 155.155635) (width 0.2) (layer "B.Cu") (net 26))
 (segment (start 207.86 153.6) (end 208.96 152.5) (width 0.2) (layer "B.Cu") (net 26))
 (segment (start 207.86 155.155635) (end 207.86 153.6) (width 0.2) (layer "B.Cu") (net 26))
 (segment (start 188.12 157.35) (end 205.665635 157.35) (width 0.2) (layer "B.Cu") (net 26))
 (segment (start 188 158.5) (end 205.5 158.5) (width 0.2) (layer "B.Cu") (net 27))
 (segment (start 205.5 158.5) (end 208.96 155.04) (width 0.2) (layer "B.Cu") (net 27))
 (segment (start 226.51 156.49) (end 213.49 156.49) (width 0.2) (layer "B.Cu") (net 4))
 (segment (start 213.49 156.49) (end 212.6 155.6) (width 0.2) (layer "B.Cu") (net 4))
 (segment (start 347.77 155) (end 228 155) (width 0.2) (layer "B.Cu") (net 4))
 (segment (start 212.6 153.6) (end 211.5 152.5) (width 0.2) (layer "B.Cu") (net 4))
 (segment (start 350 157.23) (end 347.77 155) (width 0.2) (layer "B.Cu") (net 4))
 (segment (start 212.6 155.6) (end 212.6 153.6) (width 0.2) (layer "B.Cu") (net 4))
 (segment (start 228 155) (end 226.51 156.49) (width 0.2) (layer "B.Cu") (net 4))
 (segment (start 349 158.5) (end 346 155.5) (width 0.2) (layer "B.Cu") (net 5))
 (segment (start 228.5 155.5) (end 227.16 156.84) (width 0.2) (layer "B.Cu") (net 5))
 (segment (start 213.3 156.84) (end 211.5 155.04) (width 0.2) (layer "B.Cu") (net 5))
 (segment (start 346 155.5) (end 228.5 155.5) (width 0.2) (layer "B.Cu") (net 5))
 (segment (start 227.16 156.84) (end 213.3 156.84) (width 0.2) (layer "B.Cu") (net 5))
 (segment (start 350 158.5) (end 349 158.5) (width 0.2) (layer "B.Cu") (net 5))
 (segment (start 368.29 150.25) (end 361.73 150.25) (width 0.4) (layer "F.Cu") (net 18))
 (segment (start 369 149.54) (end 368.29 150.25) (width 0.4) (layer "F.Cu") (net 18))
 (segment (start 370 150) (end 369 151) (width 0.4) (layer "F.Cu") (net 18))
 (segment (start 369 149.54) (end 368.71 149.25) (width 0.4) (layer "F.Cu") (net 18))
 (segment (start 337 150.25) (end 346.5 150.25) (width 0.4) (layer "F.Cu") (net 15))
 (segment (start 346.5 150.25) (end 347.25 149.5) (width 0.4) (layer "F.Cu") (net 15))
 (segment (start 270.04 150.5) (end 271 149.54) (width 0.4) (layer "F.Cu") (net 13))
 (segment (start 261.115 150.5) (end 270.04 150.5) (width 0.4) (layer "F.Cu") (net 13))
 (segment (start 174.36 149.96) (end 174.4 150) (width 0.4) (layer "F.Cu") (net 12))
 (segment (start 167.5 149.96) (end 174.36 149.96) (width 0.4) (layer "F.Cu") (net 12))
 (segment (start 107 150.5) (end 106 149.5) (width 0.4) (layer "F.Cu") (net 17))
 (segment (start 115.385 150.5) (end 107 150.5) (width 0.4) (layer "F.Cu") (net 17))
 (segment (start 104.34 149.96) (end 104.5 149.8) (width 0.4) (layer "F.Cu") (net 17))
 (segment (start 46.25 157.5) (end 37.21 157.5) (width 0.4) (layer "F.Cu") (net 6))
 (segment (start 37.21 157.5) (end 36.25 158.46) (width 0.4) (layer "F.Cu") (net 6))
 (segment (start 104.27 157.5) (end 103.73 158.04) (width 0.4) (layer "F.Cu") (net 22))
 (segment (start 83.46 158.04) (end 83 158.5) (width 0.4) (layer "F.Cu") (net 22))
 (segment (start 103.73 158.04) (end 83.46 158.04) (width 0.4) (layer "F.Cu") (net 22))
 (segment (start 154 157.5) (end 153 158.5) (width 0.4) (layer "F.Cu") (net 20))
 (segment (start 162 157.5) (end 154 157.5) (width 0.4) (layer "F.Cu") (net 20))
 (segment (start 254.54 158.04) (end 255 158.5) (width 0.4) (layer "F.Cu") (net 10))
 (segment (start 245.5 158) (end 245.54 158.04) (width 0.4) (layer "F.Cu") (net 10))
 (segment (start 245.54 158.04) (end 254.54 158.04) (width 0.4) (layer "F.Cu") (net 10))
 (segment (start 307 158.5) (end 306.25 157.75) (width 0.4) (layer "F.Cu") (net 9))
 (segment (start 306.25 157.75) (end 298.48 157.75) (width 0.4) (layer "F.Cu") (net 9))
 (segment (start 375.75 157.5) (end 383.04 157.5) (width 0.4) (layer "F.Cu") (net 1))
 (segment (start 383.04 157.5) (end 384 158.46) (width 0.4) (layer "F.Cu") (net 1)))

